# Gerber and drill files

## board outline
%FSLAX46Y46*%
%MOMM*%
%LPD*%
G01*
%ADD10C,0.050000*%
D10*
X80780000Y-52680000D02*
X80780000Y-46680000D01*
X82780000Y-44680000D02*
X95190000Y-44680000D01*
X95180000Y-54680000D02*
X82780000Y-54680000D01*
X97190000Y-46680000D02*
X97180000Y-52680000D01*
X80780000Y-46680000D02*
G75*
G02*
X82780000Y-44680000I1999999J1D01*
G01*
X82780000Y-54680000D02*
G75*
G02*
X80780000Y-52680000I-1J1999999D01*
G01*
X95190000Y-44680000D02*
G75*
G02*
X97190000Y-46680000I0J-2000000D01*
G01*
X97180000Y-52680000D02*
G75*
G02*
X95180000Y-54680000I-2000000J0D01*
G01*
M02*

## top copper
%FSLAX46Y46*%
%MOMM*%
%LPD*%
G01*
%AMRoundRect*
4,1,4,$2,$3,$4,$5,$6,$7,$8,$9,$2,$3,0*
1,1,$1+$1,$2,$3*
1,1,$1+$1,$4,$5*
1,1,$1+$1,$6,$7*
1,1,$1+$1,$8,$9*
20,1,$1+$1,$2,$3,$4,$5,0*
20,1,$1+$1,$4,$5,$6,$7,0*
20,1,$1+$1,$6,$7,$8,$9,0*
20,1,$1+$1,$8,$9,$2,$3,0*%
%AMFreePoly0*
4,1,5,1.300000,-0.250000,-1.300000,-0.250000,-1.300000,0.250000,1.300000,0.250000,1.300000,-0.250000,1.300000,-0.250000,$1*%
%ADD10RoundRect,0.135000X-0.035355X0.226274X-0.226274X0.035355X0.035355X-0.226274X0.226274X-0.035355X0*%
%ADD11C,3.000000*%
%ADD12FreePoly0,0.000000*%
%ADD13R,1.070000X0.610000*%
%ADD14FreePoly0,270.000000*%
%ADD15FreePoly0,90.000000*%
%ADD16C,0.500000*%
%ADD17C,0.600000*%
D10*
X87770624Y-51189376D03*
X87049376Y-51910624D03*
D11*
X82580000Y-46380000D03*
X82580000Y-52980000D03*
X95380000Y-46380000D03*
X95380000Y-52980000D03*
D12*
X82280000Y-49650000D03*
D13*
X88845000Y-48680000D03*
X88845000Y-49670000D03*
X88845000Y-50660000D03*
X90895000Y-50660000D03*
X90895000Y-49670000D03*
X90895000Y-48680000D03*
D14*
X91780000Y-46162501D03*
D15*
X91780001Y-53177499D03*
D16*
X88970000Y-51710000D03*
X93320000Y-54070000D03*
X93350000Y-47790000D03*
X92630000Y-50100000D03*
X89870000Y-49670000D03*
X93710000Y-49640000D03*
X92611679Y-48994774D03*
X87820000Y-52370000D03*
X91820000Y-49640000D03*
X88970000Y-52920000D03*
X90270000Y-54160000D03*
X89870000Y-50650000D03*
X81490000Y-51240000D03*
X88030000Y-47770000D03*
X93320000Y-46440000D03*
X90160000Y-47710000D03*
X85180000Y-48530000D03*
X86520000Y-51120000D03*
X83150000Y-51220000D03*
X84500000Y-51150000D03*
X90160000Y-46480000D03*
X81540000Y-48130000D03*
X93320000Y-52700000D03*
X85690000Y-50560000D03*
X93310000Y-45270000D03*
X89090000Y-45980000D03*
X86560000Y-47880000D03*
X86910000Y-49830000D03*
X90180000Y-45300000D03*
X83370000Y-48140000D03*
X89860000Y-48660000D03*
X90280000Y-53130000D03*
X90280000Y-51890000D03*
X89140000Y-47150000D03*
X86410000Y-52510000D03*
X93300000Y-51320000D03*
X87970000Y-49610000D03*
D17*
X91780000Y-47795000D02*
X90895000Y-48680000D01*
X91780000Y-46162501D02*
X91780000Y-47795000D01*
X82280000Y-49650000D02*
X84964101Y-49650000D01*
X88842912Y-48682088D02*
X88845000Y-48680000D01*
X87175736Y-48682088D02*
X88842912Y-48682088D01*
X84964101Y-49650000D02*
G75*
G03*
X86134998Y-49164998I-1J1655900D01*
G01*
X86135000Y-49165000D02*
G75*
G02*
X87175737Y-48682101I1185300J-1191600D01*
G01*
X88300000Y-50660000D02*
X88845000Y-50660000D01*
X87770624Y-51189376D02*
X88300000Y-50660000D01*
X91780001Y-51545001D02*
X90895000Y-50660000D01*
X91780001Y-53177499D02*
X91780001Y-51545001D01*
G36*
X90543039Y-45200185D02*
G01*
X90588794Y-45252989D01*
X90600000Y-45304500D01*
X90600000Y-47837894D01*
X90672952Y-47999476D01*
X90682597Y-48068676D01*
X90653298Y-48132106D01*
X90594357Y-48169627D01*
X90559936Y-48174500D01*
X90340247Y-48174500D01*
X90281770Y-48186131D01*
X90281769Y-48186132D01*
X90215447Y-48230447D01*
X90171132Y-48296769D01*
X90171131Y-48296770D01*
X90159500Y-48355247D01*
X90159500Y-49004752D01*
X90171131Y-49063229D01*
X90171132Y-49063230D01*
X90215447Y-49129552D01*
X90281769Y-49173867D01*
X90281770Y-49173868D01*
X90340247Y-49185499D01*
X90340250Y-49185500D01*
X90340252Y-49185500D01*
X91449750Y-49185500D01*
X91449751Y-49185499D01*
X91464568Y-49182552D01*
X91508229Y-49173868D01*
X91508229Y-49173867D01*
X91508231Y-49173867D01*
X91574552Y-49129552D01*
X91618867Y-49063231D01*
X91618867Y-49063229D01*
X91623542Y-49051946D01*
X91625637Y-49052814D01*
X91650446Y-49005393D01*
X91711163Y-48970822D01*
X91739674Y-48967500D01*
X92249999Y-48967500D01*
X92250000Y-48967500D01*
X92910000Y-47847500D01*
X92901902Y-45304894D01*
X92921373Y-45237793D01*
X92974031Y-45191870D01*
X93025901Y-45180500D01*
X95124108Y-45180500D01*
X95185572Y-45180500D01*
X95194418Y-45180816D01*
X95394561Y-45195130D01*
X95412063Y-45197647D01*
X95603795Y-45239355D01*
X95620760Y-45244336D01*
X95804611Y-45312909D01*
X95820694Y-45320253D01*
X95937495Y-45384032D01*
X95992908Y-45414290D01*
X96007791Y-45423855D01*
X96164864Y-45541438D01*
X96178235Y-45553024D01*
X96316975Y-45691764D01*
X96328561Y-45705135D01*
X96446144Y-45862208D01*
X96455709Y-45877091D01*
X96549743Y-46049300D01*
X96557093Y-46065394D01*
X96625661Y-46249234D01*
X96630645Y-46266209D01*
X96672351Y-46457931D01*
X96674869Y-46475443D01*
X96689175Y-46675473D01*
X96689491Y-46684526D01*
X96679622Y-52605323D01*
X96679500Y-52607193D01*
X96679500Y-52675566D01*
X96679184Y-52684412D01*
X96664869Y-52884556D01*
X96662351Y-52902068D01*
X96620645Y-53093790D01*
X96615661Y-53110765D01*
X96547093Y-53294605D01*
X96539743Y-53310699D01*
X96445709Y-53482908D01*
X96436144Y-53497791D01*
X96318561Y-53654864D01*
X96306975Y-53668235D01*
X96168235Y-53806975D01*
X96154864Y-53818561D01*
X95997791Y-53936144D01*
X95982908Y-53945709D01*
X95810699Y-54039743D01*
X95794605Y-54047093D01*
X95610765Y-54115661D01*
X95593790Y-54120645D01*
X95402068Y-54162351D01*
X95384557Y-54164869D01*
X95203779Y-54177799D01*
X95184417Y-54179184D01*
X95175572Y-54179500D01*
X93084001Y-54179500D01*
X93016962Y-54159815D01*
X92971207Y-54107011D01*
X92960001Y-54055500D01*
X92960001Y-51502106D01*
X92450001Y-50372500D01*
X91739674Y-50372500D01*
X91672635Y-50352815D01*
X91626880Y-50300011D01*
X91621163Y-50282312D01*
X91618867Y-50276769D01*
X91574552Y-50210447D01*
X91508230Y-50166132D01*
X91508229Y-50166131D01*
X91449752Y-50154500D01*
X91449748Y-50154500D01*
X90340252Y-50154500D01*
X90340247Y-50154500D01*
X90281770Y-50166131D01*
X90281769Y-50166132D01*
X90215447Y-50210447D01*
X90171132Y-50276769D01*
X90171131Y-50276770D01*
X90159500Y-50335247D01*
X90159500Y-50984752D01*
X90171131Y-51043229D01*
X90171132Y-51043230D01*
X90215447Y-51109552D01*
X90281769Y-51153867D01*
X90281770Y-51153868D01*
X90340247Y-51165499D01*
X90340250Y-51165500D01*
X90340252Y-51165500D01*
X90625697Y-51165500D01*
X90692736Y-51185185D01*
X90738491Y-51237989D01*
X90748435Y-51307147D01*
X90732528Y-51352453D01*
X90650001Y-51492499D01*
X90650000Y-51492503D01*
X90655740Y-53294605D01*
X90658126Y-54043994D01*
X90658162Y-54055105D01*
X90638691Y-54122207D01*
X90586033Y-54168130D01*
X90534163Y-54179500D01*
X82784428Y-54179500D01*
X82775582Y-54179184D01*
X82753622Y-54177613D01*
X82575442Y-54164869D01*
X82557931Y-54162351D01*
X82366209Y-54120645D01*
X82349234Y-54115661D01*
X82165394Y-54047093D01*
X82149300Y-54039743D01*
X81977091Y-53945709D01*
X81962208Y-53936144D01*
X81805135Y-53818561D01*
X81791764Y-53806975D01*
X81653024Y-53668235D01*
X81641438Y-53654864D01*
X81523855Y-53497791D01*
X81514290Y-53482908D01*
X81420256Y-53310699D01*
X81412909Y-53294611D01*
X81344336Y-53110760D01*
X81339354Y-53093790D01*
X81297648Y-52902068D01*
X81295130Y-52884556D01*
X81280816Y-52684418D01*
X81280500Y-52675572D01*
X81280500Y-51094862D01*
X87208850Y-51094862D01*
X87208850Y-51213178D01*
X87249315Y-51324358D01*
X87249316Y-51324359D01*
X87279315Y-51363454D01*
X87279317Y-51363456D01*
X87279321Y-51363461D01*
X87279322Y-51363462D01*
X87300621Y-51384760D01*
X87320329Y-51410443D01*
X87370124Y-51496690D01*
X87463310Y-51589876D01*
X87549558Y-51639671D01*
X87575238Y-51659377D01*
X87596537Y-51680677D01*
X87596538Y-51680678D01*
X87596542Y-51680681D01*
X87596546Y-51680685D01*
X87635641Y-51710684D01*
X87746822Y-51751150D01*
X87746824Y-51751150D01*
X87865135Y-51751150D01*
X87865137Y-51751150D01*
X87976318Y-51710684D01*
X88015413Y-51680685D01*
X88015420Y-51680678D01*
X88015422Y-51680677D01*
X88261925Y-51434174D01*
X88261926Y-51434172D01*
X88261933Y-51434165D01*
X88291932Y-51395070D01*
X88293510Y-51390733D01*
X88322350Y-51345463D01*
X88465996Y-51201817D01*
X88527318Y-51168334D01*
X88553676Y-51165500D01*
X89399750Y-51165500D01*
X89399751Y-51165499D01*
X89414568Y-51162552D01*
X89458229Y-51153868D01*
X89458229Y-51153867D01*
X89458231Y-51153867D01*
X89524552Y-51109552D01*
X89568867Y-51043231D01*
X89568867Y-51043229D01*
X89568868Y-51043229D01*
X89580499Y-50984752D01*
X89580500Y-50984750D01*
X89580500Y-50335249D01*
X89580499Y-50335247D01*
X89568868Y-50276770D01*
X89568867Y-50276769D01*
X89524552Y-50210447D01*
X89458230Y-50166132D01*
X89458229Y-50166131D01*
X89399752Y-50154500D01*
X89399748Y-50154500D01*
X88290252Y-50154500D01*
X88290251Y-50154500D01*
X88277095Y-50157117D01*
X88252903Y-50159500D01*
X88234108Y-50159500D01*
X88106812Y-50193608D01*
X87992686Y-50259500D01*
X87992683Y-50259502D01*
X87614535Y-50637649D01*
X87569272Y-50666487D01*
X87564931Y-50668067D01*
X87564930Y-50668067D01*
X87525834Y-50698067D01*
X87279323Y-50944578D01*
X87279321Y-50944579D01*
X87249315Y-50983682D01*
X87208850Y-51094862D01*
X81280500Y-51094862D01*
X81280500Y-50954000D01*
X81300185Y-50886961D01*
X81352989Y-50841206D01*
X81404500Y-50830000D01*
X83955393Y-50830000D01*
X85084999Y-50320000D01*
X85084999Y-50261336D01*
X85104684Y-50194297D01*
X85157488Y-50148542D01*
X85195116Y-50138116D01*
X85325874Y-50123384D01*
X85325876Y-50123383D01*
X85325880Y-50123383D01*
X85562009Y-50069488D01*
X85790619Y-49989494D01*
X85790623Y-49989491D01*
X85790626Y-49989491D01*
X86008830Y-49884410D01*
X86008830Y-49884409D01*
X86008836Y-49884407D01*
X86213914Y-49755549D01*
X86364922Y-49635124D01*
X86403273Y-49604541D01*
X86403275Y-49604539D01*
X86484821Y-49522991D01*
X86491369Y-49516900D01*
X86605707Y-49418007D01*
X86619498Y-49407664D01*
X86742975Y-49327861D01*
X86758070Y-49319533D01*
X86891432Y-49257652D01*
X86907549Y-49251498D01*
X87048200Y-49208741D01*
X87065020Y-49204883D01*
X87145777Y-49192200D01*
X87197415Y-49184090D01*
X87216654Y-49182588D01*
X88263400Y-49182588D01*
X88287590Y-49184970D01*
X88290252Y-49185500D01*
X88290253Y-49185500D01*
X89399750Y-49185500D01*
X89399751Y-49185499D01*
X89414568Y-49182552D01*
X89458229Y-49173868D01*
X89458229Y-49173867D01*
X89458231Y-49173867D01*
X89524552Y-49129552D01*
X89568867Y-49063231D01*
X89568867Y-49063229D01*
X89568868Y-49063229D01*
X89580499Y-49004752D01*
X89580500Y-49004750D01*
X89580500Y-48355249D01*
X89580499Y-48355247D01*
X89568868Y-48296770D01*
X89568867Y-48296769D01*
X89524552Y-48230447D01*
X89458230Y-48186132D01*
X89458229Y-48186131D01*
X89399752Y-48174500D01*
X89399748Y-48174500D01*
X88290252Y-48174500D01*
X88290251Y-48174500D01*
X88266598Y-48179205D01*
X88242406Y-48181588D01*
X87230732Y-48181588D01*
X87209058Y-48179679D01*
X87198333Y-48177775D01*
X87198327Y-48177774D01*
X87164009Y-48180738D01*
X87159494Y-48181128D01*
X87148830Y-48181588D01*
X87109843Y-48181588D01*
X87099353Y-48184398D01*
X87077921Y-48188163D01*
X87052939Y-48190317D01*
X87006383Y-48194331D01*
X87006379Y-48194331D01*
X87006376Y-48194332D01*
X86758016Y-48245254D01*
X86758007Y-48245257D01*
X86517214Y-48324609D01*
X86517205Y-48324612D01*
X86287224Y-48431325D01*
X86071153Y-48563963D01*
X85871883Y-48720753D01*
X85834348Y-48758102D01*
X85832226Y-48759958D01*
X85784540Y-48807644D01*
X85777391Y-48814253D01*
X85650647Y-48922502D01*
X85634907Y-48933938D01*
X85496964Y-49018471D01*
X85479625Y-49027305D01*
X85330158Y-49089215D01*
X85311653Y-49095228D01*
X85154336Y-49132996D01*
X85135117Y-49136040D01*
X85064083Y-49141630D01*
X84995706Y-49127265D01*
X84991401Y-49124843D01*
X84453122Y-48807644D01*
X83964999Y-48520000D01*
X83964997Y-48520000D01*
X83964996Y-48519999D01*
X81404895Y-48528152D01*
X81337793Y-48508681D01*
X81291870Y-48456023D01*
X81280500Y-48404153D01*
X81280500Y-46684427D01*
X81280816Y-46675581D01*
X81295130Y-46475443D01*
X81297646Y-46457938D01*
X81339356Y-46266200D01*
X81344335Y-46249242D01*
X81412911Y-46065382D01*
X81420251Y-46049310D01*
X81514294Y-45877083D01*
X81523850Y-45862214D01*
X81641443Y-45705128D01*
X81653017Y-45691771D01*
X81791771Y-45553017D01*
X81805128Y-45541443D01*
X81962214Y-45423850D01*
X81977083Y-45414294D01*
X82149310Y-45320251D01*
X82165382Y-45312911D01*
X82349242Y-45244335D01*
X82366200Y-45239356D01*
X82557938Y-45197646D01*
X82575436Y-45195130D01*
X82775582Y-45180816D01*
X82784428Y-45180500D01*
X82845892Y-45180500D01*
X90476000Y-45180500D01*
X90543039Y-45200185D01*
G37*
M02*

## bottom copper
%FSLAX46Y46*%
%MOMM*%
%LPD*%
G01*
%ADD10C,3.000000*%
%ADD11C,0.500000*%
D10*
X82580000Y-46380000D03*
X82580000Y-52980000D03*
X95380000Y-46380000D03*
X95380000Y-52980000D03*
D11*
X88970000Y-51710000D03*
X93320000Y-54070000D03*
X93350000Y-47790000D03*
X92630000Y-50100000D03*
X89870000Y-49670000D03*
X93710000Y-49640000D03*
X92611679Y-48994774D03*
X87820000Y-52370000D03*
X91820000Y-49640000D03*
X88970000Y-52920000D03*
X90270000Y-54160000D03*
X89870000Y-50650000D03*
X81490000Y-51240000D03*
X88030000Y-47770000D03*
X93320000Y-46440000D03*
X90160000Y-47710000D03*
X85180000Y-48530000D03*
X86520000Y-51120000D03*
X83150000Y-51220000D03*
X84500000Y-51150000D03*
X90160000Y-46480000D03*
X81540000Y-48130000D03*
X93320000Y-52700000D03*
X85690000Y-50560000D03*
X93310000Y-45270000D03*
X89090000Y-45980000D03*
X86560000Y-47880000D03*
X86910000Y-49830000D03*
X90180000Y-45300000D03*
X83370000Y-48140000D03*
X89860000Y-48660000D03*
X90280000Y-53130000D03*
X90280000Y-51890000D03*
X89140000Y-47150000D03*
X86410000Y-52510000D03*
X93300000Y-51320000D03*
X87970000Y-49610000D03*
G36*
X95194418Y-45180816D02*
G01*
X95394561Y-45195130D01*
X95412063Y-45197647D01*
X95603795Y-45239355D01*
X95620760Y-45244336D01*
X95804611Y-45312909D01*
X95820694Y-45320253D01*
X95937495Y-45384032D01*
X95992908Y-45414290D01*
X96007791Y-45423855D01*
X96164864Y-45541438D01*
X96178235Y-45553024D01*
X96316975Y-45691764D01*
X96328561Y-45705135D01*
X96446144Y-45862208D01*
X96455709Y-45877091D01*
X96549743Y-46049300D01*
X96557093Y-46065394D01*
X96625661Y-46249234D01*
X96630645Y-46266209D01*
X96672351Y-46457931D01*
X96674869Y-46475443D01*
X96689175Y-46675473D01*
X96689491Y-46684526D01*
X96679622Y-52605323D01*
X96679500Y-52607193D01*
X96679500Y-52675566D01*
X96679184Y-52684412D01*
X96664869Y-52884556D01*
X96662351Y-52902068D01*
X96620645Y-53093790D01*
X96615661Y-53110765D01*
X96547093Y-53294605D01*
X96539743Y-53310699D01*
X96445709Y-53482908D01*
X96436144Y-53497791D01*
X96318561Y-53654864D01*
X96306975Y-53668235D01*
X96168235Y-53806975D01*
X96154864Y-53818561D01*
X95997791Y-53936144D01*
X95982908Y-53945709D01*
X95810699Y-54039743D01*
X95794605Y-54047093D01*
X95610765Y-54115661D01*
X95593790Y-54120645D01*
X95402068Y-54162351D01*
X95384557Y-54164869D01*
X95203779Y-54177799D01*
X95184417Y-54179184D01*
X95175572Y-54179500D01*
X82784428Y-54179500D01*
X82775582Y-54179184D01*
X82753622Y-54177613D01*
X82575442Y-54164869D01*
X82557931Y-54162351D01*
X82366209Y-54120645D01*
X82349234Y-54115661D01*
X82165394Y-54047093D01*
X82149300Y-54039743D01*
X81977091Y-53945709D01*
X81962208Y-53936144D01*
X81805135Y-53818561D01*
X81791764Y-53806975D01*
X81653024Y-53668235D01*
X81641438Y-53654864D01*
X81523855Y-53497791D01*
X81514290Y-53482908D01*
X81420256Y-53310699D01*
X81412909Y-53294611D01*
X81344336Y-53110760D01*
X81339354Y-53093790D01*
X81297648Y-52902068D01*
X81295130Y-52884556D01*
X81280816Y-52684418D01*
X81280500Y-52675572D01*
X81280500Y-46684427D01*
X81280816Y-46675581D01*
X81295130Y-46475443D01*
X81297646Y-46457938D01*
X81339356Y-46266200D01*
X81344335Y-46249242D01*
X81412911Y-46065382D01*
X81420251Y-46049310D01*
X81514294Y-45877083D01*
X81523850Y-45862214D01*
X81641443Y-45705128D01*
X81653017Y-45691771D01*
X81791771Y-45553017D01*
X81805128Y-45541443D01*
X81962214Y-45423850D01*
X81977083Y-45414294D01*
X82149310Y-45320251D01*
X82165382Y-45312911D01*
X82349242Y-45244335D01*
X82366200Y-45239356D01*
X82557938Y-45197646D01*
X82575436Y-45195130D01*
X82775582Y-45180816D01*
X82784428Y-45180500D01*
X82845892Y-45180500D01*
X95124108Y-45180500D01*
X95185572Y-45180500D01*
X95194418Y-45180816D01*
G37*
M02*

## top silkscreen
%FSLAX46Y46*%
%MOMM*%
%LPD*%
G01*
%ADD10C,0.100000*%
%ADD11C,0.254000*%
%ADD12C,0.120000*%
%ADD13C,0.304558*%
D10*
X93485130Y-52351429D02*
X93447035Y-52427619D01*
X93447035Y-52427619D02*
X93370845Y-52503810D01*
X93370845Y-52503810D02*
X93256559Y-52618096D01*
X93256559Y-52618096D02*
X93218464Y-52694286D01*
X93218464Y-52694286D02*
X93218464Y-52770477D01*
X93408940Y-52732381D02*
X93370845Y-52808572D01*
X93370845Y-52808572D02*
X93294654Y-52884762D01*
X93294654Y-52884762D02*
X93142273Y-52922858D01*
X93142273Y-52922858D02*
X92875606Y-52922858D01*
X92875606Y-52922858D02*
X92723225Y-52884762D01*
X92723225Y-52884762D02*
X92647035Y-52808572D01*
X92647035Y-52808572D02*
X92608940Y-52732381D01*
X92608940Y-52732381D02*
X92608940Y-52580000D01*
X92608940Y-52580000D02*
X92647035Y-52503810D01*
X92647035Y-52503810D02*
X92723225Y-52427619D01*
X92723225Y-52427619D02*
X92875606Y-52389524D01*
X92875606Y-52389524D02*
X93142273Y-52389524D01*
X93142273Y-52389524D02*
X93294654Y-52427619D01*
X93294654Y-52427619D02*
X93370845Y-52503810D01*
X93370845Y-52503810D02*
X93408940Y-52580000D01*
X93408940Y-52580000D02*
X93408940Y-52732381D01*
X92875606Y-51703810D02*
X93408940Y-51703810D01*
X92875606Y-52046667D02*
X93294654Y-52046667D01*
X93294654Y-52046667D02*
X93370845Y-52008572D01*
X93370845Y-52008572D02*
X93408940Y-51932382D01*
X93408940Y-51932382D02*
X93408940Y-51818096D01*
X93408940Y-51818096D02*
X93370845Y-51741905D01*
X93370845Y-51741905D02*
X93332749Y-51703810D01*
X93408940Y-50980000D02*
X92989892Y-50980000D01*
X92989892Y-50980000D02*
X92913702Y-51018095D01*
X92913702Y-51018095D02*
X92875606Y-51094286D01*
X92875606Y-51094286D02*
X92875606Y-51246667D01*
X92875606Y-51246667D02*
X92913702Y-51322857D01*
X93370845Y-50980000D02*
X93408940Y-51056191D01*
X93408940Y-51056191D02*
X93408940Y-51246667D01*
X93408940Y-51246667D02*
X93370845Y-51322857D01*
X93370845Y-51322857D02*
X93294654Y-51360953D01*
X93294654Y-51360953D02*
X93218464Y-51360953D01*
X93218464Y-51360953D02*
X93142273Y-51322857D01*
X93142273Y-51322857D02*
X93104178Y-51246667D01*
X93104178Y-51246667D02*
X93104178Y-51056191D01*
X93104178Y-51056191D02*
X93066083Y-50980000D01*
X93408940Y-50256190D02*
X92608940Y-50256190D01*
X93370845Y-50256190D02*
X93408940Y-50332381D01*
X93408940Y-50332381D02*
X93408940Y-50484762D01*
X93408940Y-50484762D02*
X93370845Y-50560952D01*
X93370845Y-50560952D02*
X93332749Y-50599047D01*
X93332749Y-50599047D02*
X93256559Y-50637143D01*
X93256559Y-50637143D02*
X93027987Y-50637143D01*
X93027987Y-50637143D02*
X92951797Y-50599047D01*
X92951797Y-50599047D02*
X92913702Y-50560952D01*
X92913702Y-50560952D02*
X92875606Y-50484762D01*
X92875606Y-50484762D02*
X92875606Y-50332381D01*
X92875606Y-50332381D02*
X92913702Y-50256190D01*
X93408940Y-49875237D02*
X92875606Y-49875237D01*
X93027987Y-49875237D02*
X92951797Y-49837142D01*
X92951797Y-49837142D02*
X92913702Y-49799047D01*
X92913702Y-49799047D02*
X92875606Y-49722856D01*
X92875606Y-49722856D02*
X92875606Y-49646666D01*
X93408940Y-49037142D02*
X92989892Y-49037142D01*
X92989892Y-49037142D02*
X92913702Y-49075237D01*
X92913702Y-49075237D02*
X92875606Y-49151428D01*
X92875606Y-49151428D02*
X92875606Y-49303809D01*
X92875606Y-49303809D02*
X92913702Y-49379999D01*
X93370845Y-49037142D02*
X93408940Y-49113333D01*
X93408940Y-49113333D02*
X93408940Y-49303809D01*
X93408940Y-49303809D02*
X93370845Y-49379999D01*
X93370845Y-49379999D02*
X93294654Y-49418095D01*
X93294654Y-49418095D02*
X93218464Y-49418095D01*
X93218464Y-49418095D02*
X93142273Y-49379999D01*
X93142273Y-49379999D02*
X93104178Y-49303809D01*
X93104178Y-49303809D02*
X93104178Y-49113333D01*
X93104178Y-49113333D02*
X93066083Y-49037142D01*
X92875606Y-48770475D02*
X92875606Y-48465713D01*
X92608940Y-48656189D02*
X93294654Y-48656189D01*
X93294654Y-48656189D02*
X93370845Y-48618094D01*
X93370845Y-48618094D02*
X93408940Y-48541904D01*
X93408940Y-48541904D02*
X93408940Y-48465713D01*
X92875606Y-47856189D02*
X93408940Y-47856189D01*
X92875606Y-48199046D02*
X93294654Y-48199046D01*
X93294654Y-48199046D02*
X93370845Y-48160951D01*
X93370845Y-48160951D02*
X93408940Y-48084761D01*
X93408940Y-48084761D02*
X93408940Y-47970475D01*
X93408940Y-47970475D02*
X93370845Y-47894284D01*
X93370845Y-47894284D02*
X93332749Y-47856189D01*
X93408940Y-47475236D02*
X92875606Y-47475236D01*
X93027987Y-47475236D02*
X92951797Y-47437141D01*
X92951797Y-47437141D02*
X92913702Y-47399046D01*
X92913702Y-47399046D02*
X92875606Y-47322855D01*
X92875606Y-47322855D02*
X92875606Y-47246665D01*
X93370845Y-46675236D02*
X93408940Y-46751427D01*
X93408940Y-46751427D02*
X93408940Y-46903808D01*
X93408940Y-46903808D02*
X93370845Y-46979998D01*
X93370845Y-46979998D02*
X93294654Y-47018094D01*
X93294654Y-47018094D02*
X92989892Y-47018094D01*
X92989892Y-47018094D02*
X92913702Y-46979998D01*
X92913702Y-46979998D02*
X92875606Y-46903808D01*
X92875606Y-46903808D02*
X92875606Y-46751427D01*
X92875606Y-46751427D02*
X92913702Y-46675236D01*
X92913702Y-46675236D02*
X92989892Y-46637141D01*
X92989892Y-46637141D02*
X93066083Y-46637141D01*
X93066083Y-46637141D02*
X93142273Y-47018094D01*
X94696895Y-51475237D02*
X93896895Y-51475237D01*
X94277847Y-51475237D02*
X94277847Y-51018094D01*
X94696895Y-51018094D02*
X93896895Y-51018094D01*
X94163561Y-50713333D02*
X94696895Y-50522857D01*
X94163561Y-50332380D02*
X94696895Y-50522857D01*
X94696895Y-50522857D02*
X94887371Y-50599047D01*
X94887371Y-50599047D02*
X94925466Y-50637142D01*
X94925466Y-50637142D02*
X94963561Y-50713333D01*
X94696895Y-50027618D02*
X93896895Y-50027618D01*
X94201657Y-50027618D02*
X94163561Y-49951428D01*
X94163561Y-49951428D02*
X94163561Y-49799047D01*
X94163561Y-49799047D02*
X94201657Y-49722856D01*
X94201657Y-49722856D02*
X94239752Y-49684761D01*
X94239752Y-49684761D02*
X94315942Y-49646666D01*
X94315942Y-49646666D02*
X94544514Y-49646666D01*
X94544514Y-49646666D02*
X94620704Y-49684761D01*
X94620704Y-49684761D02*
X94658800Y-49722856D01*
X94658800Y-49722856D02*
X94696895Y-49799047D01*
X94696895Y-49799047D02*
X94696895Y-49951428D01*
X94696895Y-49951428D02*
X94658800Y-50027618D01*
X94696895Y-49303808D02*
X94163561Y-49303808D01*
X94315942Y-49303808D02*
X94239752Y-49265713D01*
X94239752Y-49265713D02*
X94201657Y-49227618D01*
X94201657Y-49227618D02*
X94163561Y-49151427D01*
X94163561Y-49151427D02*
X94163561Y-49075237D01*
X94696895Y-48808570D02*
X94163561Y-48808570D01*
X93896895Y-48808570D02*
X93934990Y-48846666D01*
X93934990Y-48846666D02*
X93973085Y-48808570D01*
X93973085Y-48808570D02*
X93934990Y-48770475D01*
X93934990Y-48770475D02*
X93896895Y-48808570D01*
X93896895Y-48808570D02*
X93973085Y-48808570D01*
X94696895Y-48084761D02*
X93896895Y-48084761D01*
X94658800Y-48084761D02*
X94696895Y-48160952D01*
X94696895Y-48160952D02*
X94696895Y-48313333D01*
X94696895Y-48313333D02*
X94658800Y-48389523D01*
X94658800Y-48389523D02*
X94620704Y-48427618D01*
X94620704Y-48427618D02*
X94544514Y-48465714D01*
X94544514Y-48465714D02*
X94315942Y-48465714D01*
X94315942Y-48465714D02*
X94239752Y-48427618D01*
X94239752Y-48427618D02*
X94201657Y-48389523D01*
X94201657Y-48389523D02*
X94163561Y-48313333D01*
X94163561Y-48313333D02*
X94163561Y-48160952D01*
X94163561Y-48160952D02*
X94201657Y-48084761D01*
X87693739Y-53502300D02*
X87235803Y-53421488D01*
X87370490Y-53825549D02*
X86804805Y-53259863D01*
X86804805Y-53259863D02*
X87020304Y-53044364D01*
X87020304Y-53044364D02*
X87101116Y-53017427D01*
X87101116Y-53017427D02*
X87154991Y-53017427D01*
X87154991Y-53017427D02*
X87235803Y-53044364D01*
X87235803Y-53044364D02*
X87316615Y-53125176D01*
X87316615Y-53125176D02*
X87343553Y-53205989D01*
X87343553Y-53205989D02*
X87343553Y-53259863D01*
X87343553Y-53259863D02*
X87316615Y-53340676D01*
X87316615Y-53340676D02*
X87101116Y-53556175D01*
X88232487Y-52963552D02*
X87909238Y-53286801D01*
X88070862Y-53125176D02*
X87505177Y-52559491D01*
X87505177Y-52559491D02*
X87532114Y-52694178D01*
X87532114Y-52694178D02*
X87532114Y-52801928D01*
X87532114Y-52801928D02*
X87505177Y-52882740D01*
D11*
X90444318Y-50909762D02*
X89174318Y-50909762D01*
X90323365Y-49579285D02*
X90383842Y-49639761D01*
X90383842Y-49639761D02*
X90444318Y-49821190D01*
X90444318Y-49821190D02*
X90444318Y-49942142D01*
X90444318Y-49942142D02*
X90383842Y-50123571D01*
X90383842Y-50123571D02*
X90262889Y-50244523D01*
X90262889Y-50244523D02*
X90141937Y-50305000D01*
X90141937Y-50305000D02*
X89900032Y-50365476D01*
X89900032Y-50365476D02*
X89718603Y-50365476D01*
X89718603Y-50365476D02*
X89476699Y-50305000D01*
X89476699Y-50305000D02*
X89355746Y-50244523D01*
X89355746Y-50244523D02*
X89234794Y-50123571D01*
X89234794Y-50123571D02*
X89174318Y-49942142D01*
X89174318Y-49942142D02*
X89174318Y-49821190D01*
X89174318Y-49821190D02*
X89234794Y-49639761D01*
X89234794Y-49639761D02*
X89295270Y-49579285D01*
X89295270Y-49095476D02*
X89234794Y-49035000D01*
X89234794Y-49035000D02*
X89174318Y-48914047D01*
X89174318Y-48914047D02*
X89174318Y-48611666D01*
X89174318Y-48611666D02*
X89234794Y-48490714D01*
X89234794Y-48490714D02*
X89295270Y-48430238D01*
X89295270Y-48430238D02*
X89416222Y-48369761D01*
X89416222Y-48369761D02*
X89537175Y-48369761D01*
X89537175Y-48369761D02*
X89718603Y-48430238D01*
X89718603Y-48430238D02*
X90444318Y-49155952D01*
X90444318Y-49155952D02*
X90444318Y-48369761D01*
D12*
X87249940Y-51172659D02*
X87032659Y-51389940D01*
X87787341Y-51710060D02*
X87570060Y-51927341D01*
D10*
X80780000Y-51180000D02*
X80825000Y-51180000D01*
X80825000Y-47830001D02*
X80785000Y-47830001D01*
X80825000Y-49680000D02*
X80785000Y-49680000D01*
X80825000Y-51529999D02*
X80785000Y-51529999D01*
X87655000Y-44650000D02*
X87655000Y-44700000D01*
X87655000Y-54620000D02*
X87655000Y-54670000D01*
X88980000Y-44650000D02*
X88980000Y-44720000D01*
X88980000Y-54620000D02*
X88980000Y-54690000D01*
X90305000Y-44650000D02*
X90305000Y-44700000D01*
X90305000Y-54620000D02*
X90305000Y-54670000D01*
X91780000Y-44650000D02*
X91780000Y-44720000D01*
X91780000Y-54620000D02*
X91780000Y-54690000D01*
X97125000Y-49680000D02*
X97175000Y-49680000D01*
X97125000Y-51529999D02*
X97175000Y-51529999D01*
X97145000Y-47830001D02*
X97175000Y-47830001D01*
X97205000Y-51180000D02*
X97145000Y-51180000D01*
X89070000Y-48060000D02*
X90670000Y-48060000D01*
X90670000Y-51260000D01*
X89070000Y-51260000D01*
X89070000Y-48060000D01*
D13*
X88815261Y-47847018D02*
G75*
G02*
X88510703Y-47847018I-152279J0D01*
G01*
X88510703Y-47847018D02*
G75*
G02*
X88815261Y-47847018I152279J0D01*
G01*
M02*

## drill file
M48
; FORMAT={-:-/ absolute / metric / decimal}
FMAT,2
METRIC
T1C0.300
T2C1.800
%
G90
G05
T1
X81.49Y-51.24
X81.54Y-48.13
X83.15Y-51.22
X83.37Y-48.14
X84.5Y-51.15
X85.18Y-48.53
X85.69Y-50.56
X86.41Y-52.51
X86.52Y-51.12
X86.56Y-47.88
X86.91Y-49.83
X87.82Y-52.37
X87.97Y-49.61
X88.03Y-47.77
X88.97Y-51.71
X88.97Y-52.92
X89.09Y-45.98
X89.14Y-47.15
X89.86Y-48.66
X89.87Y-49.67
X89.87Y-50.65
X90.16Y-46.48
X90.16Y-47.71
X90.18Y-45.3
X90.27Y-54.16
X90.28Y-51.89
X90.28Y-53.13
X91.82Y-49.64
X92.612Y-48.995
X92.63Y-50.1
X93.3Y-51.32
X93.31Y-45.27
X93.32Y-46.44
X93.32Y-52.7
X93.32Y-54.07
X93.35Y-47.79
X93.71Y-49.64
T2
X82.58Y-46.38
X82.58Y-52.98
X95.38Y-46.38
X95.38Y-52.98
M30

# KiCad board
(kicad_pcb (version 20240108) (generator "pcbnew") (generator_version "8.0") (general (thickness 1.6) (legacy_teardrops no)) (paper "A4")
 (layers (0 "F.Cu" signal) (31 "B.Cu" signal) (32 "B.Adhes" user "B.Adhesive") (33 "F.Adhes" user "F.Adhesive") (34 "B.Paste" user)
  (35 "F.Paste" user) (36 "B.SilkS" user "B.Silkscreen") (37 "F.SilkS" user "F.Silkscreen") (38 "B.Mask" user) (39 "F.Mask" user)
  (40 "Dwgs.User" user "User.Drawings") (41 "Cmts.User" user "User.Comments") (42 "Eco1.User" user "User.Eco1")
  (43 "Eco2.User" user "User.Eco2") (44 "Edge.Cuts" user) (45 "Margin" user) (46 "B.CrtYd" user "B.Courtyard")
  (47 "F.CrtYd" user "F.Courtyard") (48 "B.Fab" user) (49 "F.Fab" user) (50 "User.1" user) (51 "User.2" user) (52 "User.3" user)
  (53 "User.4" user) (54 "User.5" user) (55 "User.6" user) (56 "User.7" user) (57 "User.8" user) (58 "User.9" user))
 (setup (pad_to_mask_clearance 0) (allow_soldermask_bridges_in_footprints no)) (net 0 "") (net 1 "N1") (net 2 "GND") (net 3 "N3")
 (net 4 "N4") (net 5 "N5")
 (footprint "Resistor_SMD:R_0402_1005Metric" (layer "F.Cu") (at 87.41 51.55 -135)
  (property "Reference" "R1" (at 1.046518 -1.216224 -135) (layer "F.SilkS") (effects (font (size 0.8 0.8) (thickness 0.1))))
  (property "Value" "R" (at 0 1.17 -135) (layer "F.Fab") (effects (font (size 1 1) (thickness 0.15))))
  (fp_line (start -0.153641 0.38) (end 0.153641 0.38) (stroke (width 0.12) (type solid)) (layer "F.SilkS"))
  (fp_line (start -0.153641 -0.38) (end 0.153641 -0.38) (stroke (width 0.12) (type solid)) (layer "F.SilkS"))
  (pad "1" smd roundrect (at -0.509999 0 225) (size 0.54 0.64) (layers "F.Cu" "F.Paste" "F.Mask") (roundrect_rratio 0.25) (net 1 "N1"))
  (pad "2" smd roundrect (at 0.509999 0 225) (size 0.54 0.64) (layers "F.Cu" "F.Paste" "F.Mask") (roundrect_rratio 0.25) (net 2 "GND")))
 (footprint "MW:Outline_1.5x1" (layer "F.Cu") (at 88.98 49.68)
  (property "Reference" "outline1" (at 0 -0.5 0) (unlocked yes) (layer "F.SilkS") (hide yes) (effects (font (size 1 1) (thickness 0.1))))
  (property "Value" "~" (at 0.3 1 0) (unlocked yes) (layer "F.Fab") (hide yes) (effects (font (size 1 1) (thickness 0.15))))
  (fp_line (start -8.2 1.5) (end -8.155 1.5) (stroke (width 0.1) (type default)) (layer "F.SilkS"))
  (fp_line (start -8.155 -1.849999) (end -8.195 -1.849999) (stroke (width 0.1) (type default)) (layer "F.SilkS"))
  (fp_line (start -8.155 0) (end -8.195 0) (stroke (width 0.1) (type default)) (layer "F.SilkS"))
  (fp_line (start -8.155 1.849999) (end -8.195 1.849999) (stroke (width 0.1) (type default)) (layer "F.SilkS"))
  (fp_line (start -1.325 -5.03) (end -1.325 -4.98) (stroke (width 0.1) (type default)) (layer "F.SilkS"))
  (fp_line (start -1.325 4.94) (end -1.325 4.99) (stroke (width 0.1) (type default)) (layer "F.SilkS"))
  (fp_line (start 0 -5.03) (end 0 -4.96) (stroke (width 0.1) (type default)) (layer "F.SilkS"))
  (fp_line (start 0 4.94) (end 0 5.01) (stroke (width 0.1) (type default)) (layer "F.SilkS"))
  (fp_line (start 1.325 -5.03) (end 1.325 -4.98) (stroke (width 0.1) (type default)) (layer "F.SilkS"))
  (fp_line (start 1.325 4.94) (end 1.325 4.99) (stroke (width 0.1) (type default)) (layer "F.SilkS"))
  (fp_line (start 2.8 -5.03) (end 2.8 -4.96) (stroke (width 0.1) (type default)) (layer "F.SilkS"))
  (fp_line (start 2.8 4.94) (end 2.8 5.01) (stroke (width 0.1) (type default)) (layer "F.SilkS"))
  (fp_line (start 8.145 0) (end 8.195 0) (stroke (width 0.1) (type default)) (layer "F.SilkS"))
  (fp_line (start 8.145 1.849999) (end 8.195 1.849999) (stroke (width 0.1) (type default)) (layer "F.SilkS"))
  (fp_line (start 8.165 -1.849999) (end 8.195 -1.849999) (stroke (width 0.1) (type default)) (layer "F.SilkS"))
  (fp_line (start 8.225 1.5) (end 8.165 1.5) (stroke (width 0.1) (type default)) (layer "F.SilkS"))
  (fp_line (start -8.2 3) (end -8.2 -3) (stroke (width 0.05) (type default)) (layer "Edge.Cuts"))
  (fp_line (start -6.2 -5) (end 6.21 -5) (stroke (width 0.05) (type default)) (layer "Edge.Cuts"))
  (fp_line (start 6.2 5) (end -6.2 5) (stroke (width 0.05) (type default)) (layer "Edge.Cuts"))
  (fp_line (start 8.21 -3) (end 8.2 3) (stroke (width 0.05) (type default)) (layer "Edge.Cuts"))
  (fp_arc (start -8.2 -3) (mid -7.614214 -4.414214) (end -6.2 -5) (stroke (width 0.05) (type default)) (layer "Edge.Cuts"))
  (fp_arc (start -6.2 5) (mid -7.614214 4.414214) (end -8.2 3) (stroke (width 0.05) (type default)) (layer "Edge.Cuts"))
  (fp_arc (start 6.21 -5) (mid 7.624214 -4.414214) (end 8.21 -3) (stroke (width 0.05) (type default)) (layer "Edge.Cuts"))
  (fp_arc (start 8.2 3) (mid 7.614214 4.414214) (end 6.2 5) (stroke (width 0.05) (type default)) (layer "Edge.Cuts"))
  (pad "1" thru_hole circle (at -6.4 -3.3) (size 3 3) (drill 1.8) (layers "*.Cu" "*.Mask") (remove_unused_layers no) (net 2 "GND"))
  (pad "1" thru_hole circle (at -6.4 3.3) (size 3 3) (drill 1.8) (layers "*.Cu" "*.Mask") (remove_unused_layers no) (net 2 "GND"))
  (pad "1" thru_hole circle (at 6.4 -3.3) (size 3 3) (drill 1.8) (layers "*.Cu" "*.Mask") (remove_unused_layers no) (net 2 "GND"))
  (pad "1" thru_hole circle (at 6.4 3.3) (size 3 3) (drill 1.8) (layers "*.Cu" "*.Mask") (remove_unused_layers no) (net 2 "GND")))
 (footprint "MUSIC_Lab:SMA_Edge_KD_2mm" (layer "F.Cu") (at 83.004999 49.71)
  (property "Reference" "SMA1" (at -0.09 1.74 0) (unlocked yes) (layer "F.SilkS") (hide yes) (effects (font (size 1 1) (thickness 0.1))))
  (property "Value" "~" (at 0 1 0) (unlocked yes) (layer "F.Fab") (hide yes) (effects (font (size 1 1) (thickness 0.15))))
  (pad "1" smd custom (at -0.724999 -0.06) (size 2.6 0.5) (layers "F.Cu" "F.Paste" "F.Mask") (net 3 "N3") (thermal_bridge_angle 45)
   (options (clearance outline) (anchor rect)) (primitives))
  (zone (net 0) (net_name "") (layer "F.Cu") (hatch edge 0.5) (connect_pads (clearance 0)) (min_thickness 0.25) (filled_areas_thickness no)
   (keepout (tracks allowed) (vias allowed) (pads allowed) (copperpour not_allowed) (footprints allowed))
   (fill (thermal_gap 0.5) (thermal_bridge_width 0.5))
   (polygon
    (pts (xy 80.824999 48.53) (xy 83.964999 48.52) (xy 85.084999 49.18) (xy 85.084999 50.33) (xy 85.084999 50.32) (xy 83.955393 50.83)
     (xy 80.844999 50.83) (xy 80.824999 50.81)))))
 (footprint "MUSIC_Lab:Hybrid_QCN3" (layer "F.Cu") (at 89.87 49.67 -90)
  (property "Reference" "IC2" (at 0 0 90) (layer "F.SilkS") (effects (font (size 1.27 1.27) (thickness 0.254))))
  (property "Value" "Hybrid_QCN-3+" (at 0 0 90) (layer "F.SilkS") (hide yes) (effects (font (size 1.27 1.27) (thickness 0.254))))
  (fp_rect (start -1.61 -0.8) (end 1.59 0.8) (stroke (width 0.1) (type default)) (fill none) (layer "F.SilkS"))
  (fp_circle (center -1.822982 1.207018) (end -1.568424 1.207018) (stroke (width 0.1) (type solid)) (fill solid) (layer "F.SilkS"))
  (pad "1" smd rect (at -0.99 1.025 270) (size 0.61 1.07) (layers "F.Cu" "F.Paste" "F.Mask") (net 3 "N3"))
  (pad "2" smd rect (at 0 1.025 270) (size 0.61 1.07) (layers "F.Cu" "F.Paste" "F.Mask") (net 2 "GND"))
  (pad "3" smd rect (at 0.99 1.025 270) (size 0.61 1.07) (layers "F.Cu" "F.Paste" "F.Mask") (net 1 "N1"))
  (pad "4" smd rect (at 0.99 -1.025 270) (size 0.61 1.07) (layers "F.Cu" "F.Paste" "F.Mask") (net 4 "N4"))
  (pad "5" smd rect (at 0 -1.025 270) (size 0.61 1.07) (layers "F.Cu" "F.Paste" "F.Mask") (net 2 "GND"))
  (pad "6" smd rect (at -0.99 -1.025 270) (size 0.61 1.07) (layers "F.Cu" "F.Paste" "F.Mask") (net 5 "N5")))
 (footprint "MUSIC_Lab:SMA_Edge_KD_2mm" (layer "F.Cu") (at 91.72 46.8875 -90)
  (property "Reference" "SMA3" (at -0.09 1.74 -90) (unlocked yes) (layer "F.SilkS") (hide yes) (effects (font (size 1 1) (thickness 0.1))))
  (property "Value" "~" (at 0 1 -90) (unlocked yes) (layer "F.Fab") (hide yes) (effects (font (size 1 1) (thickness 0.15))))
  (pad "1" smd custom (at -0.724999 -0.06 270) (size 2.6 0.5) (layers "F.Cu" "F.Paste" "F.Mask") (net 5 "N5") (thermal_bridge_angle 45)
   (options (clearance outline) (anchor rect)) (primitives))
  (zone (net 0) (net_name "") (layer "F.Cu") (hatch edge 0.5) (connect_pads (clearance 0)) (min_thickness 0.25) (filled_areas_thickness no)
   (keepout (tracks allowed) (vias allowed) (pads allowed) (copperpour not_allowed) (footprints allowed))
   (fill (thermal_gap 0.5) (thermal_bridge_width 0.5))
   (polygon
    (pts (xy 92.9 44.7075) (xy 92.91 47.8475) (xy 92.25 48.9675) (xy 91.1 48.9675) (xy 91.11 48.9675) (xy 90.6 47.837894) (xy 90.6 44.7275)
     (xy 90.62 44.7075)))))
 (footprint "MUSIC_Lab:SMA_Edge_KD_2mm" (layer "F.Cu") (at 91.840001 52.4525 90)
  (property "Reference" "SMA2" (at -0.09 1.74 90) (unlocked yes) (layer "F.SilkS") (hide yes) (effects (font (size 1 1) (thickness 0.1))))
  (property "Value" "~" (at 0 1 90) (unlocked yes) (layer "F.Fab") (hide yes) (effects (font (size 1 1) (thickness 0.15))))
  (pad "1" smd custom (at -0.724999 -0.06 90) (size 2.6 0.5) (layers "F.Cu" "F.Paste" "F.Mask") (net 4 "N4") (thermal_bridge_angle 45)
   (options (clearance outline) (anchor rect)) (primitives))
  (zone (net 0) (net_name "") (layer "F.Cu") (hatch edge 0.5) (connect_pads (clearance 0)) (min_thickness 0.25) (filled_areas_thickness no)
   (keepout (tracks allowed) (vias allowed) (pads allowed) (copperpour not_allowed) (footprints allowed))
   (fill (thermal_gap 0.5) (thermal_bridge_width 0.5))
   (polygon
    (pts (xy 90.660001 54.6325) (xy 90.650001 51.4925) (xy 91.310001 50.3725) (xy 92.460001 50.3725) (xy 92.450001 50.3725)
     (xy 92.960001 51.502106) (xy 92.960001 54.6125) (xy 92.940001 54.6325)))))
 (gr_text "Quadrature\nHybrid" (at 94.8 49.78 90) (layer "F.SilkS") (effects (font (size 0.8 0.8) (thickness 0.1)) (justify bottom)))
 (via (at 88.97 51.71) (size 0.5) (drill 0.3) (layers "F.Cu" "B.Cu") (free yes) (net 2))
 (via (at 93.32 54.07) (size 0.5) (drill 0.3) (layers "F.Cu" "B.Cu") (free yes) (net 2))
 (via (at 93.35 47.79) (size 0.5) (drill 0.3) (layers "F.Cu" "B.Cu") (free yes) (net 2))
 (via (at 92.63 50.1) (size 0.5) (drill 0.3) (layers "F.Cu" "B.Cu") (free yes) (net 2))
 (via (at 89.87 49.67) (size 0.5) (drill 0.3) (layers "F.Cu" "B.Cu") (free yes) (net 2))
 (via (at 93.71 49.64) (size 0.5) (drill 0.3) (layers "F.Cu" "B.Cu") (free yes) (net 2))
 (via (at 92.611679 48.994774) (size 0.5) (drill 0.3) (layers "F.Cu" "B.Cu") (free yes) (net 2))
 (via (at 87.82 52.37) (size 0.5) (drill 0.3) (layers "F.Cu" "B.Cu") (free yes) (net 2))
 (via (at 91.82 49.64) (size 0.5) (drill 0.3) (layers "F.Cu" "B.Cu") (free yes) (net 2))
 (via (at 88.97 52.92) (size 0.5) (drill 0.3) (layers "F.Cu" "B.Cu") (free yes) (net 2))
 (via (at 90.27 54.16) (size 0.5) (drill 0.3) (layers "F.Cu" "B.Cu") (free yes) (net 2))
 (via (at 89.87 50.65) (size 0.5) (drill 0.3) (layers "F.Cu" "B.Cu") (free yes) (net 2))
 (via (at 81.49 51.24) (size 0.5) (drill 0.3) (layers "F.Cu" "B.Cu") (free yes) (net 2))
 (via (at 88.03 47.77) (size 0.5) (drill 0.3) (layers "F.Cu" "B.Cu") (free yes) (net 2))
 (via (at 93.32 46.44) (size 0.5) (drill 0.3) (layers "F.Cu" "B.Cu") (free yes) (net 2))
 (via (at 90.16 47.71) (size 0.5) (drill 0.3) (layers "F.Cu" "B.Cu") (free yes) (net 2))
 (via (at 85.18 48.53) (size 0.5) (drill 0.3) (layers "F.Cu" "B.Cu") (free yes) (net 2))
 (via (at 86.52 51.12) (size 0.5) (drill 0.3) (layers "F.Cu" "B.Cu") (free yes) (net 2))
 (via (at 83.15 51.22) (size 0.5) (drill 0.3) (layers "F.Cu" "B.Cu") (free yes) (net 2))
 (via (at 84.5 51.15) (size 0.5) (drill 0.3) (layers "F.Cu" "B.Cu") (free yes) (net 2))
 (via (at 90.16 46.48) (size 0.5) (drill 0.3) (layers "F.Cu" "B.Cu") (free yes) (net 2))
 (via (at 81.54 48.13) (size 0.5) (drill 0.3) (layers "F.Cu" "B.Cu") (free yes) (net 2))
 (via (at 93.32 52.7) (size 0.5) (drill 0.3) (layers "F.Cu" "B.Cu") (free yes) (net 2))
 (via (at 85.69 50.56) (size 0.5) (drill 0.3) (layers "F.Cu" "B.Cu") (free yes) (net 2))
 (via (at 93.31 45.27) (size 0.5) (drill 0.3) (layers "F.Cu" "B.Cu") (free yes) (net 2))
 (via (at 89.09 45.98) (size 0.5) (drill 0.3) (layers "F.Cu" "B.Cu") (free yes) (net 2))
 (via (at 86.56 47.88) (size 0.5) (drill 0.3) (layers "F.Cu" "B.Cu") (free yes) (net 2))
 (via (at 86.91 49.83) (size 0.5) (drill 0.3) (layers "F.Cu" "B.Cu") (free yes) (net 2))
 (via (at 90.18 45.3) (size 0.5) (drill 0.3) (layers "F.Cu" "B.Cu") (free yes) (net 2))
 (via (at 83.37 48.14) (size 0.5) (drill 0.3) (layers "F.Cu" "B.Cu") (free yes) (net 2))
 (via (at 89.86 48.66) (size 0.5) (drill 0.3) (layers "F.Cu" "B.Cu") (free yes) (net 2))
 (via (at 90.28 53.13) (size 0.5) (drill 0.3) (layers "F.Cu" "B.Cu") (free yes) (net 2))
 (via (at 90.28 51.89) (size 0.5) (drill 0.3) (layers "F.Cu" "B.Cu") (free yes) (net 2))
 (via (at 89.14 47.15) (size 0.5) (drill 0.3) (layers "F.Cu" "B.Cu") (free yes) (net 2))
 (via (at 86.41 52.51) (size 0.5) (drill 0.3) (layers "F.Cu" "B.Cu") (free yes) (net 2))
 (via (at 93.3 51.32) (size 0.5) (drill 0.3) (layers "F.Cu" "B.Cu") (free yes) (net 2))
 (via (at 87.97 49.61) (size 0.5) (drill 0.3) (layers "F.Cu" "B.Cu") (free yes) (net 2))
 (segment (start 91.78 47.795) (end 90.895 48.68) (width 0.6) (layer "F.Cu") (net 5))
 (segment (start 91.78 46.162501) (end 91.78 47.795) (width 0.6) (layer "F.Cu") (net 5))
 (segment (start 82.28 49.65) (end 84.964101 49.65) (width 0.6) (layer "F.Cu") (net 3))
 (segment (start 88.842912 48.682088) (end 88.845 48.68) (width 0.6) (layer "F.Cu") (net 3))
 (segment (start 87.175736 48.682088) (end 88.842912 48.682088) (width 0.6) (layer "F.Cu") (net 3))
 (arc (start 84.964101 49.65) (mid 85.597789 49.523952) (end 86.135 49.165) (width 0.6) (layer "F.Cu") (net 3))
 (arc (start 86.135 49.165) (mid 86.612637 48.832105) (end 87.175736 48.682088) (width 0.6) (layer "F.Cu") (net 3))
 (segment (start 88.3 50.66) (end 88.845 50.66) (width 0.6) (layer "F.Cu") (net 1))
 (segment (start 87.770624 51.189376) (end 88.3 50.66) (width 0.6) (layer "F.Cu") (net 1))
 (segment (start 91.780001 51.545001) (end 90.895 50.66) (width 0.6) (layer "F.Cu") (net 4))
 (segment (start 91.780001 53.177499) (end 91.780001 51.545001) (width 0.6) (layer "F.Cu") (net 4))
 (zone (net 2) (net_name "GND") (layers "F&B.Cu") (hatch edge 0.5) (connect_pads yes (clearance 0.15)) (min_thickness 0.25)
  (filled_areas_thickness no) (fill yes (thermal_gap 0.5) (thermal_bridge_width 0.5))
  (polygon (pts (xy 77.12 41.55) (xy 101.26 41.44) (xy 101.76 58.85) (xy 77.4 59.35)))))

